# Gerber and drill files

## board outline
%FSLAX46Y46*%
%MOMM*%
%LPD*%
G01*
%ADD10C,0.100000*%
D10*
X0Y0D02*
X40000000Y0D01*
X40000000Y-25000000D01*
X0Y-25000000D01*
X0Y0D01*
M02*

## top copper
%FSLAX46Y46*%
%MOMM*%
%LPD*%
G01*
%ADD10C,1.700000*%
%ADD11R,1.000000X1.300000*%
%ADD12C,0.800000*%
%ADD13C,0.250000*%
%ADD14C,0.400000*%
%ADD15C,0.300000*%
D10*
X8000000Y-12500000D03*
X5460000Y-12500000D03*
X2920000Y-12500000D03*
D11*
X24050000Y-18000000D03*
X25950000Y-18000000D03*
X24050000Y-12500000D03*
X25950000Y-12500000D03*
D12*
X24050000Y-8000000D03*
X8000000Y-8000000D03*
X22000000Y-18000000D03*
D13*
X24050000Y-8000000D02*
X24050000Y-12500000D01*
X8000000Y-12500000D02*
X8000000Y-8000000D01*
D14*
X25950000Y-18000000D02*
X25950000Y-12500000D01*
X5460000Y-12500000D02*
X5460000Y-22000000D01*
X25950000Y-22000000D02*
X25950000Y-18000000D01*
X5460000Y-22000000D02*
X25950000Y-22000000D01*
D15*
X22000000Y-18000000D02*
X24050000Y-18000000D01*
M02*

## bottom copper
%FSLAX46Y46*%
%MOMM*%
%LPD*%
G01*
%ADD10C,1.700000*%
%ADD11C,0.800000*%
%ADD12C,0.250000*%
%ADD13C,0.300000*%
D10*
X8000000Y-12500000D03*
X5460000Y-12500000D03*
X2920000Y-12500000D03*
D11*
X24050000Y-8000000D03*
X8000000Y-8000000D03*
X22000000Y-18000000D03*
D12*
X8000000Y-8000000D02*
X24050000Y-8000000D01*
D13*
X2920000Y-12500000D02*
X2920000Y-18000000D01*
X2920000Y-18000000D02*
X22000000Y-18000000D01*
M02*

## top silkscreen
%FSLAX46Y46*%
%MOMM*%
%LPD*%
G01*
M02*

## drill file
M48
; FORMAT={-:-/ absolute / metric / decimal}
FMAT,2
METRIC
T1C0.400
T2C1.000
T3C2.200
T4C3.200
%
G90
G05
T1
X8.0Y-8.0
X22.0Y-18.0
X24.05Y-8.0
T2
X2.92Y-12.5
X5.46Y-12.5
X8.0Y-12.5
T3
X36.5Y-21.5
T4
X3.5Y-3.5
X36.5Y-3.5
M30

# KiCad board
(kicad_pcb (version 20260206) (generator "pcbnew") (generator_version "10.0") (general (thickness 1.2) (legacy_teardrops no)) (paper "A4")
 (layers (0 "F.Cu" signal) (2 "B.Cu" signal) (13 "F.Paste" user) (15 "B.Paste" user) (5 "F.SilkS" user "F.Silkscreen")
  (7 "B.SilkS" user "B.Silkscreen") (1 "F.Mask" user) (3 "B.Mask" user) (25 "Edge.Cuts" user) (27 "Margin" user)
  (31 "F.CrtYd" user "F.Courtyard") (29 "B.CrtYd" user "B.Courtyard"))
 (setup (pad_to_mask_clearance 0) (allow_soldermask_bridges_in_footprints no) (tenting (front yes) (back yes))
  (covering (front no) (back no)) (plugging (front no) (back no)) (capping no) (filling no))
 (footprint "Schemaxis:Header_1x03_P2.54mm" (layer "F.Cu") (at 8 12.5 -90)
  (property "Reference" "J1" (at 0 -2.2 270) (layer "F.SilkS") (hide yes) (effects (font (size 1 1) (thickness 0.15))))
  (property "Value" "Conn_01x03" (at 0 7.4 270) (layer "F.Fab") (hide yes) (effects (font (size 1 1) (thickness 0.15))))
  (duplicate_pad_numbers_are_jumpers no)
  (pad "1" thru_hole circle (at 0 0 270) (size 1.7 1.7) (drill 1) (layers "*.Cu" "*.Mask") (remove_unused_layers no) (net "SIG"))
  (pad "2" thru_hole circle (at 0 2.54 270) (size 1.7 1.7) (drill 1) (layers "*.Cu" "*.Mask") (remove_unused_layers no) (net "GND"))
  (pad "3" thru_hole circle (at 0 5.08 270) (size 1.7 1.7) (drill 1) (layers "*.Cu" "*.Mask") (remove_unused_layers no) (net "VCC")))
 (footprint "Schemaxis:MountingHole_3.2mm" (layer "F.Cu") (at 36.5 3.5)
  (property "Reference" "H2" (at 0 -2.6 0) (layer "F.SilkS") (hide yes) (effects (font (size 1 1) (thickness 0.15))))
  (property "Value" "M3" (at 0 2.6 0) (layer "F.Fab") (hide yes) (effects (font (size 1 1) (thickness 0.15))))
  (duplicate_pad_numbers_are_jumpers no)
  (pad "" np_thru_hole circle (at 0 0) (size 3.2 3.2) (drill 3.2) (layers "*.Cu" "*.Mask")))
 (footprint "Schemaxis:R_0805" (layer "F.Cu") (at 25 18)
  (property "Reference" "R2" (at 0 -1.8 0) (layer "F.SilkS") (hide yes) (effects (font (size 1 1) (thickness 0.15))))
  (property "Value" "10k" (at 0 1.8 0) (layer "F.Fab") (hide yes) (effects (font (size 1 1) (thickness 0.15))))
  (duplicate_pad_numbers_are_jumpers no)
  (pad "1" smd rect (at -0.95 0) (size 1 1.3) (layers "F.Cu" "F.Mask" "F.Paste") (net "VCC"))
  (pad "2" smd rect (at 0.95 0) (size 1 1.3) (layers "F.Cu" "F.Mask" "F.Paste") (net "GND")))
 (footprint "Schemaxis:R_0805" (layer "F.Cu") (at 25 12.5)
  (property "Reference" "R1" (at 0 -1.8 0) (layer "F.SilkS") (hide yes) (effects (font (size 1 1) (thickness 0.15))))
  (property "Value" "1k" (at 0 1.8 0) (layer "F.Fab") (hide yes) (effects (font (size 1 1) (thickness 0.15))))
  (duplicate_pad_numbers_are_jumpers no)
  (pad "1" smd rect (at -0.95 0) (size 1 1.3) (layers "F.Cu" "F.Mask" "F.Paste") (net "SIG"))
  (pad "2" smd rect (at 0.95 0) (size 1 1.3) (layers "F.Cu" "F.Mask" "F.Paste") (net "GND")))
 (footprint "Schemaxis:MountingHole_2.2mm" (layer "F.Cu") (at 36.5 21.5)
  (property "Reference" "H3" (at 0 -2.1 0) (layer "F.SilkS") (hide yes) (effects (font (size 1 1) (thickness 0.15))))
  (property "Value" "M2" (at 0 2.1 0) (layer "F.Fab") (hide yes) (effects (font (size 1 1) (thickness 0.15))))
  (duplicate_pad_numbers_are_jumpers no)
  (pad "" np_thru_hole circle (at 0 0) (size 2.2 2.2) (drill 2.2) (layers "*.Cu" "*.Mask")))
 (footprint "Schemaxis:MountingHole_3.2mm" (layer "F.Cu") (at 3.5 3.5)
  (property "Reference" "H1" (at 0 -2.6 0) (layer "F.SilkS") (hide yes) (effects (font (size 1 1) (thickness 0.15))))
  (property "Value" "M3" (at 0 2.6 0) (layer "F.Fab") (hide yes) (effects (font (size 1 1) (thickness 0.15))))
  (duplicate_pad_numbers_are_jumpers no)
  (pad "" np_thru_hole circle (at 0 0) (size 3.2 3.2) (drill 3.2) (layers "*.Cu" "*.Mask")))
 (gr_rect (start 0 0) (end 40 25) (stroke (width 0.1) (type default)) (fill no) (layer "Edge.Cuts"))
 (segment (start 24.05 8) (end 24.05 12.5) (width 0.25) (layer "F.Cu") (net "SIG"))
 (segment (start 8 12.5) (end 8 8) (width 0.25) (layer "F.Cu") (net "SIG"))
 (via (at 24.05 8) (size 0.8) (drill 0.4) (layers "F.Cu" "B.Cu") (capping no) (covering (front no) (back no))
  (plugging (front no) (back no)) (filling no) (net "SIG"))
 (via (at 8 8) (size 0.8) (drill 0.4) (layers "F.Cu" "B.Cu") (capping no) (covering (front no) (back no)) (plugging (front no) (back no))
  (filling no) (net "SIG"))
 (segment (start 8 8) (end 24.05 8) (width 0.25) (layer "B.Cu") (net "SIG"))
 (segment (start 25.95 18) (end 25.95 12.5) (width 0.4) (layer "F.Cu") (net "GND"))
 (segment (start 5.46 12.5) (end 5.46 22) (width 0.4) (layer "F.Cu") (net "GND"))
 (segment (start 25.95 22) (end 25.95 18) (width 0.4) (layer "F.Cu") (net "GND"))
 (segment (start 5.46 22) (end 25.95 22) (width 0.4) (layer "F.Cu") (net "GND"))
 (segment (start 22 18) (end 24.05 18) (width 0.3) (layer "F.Cu") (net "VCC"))
 (via (at 22 18) (size 0.8) (drill 0.4) (layers "F.Cu" "B.Cu") (capping no) (covering (front no) (back no)) (plugging (front no) (back no))
  (filling no) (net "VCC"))
 (segment (start 2.92 12.5) (end 2.92 18) (width 0.3) (layer "B.Cu") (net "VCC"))
 (segment (start 2.92 18) (end 22 18) (width 0.3) (layer "B.Cu") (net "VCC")))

